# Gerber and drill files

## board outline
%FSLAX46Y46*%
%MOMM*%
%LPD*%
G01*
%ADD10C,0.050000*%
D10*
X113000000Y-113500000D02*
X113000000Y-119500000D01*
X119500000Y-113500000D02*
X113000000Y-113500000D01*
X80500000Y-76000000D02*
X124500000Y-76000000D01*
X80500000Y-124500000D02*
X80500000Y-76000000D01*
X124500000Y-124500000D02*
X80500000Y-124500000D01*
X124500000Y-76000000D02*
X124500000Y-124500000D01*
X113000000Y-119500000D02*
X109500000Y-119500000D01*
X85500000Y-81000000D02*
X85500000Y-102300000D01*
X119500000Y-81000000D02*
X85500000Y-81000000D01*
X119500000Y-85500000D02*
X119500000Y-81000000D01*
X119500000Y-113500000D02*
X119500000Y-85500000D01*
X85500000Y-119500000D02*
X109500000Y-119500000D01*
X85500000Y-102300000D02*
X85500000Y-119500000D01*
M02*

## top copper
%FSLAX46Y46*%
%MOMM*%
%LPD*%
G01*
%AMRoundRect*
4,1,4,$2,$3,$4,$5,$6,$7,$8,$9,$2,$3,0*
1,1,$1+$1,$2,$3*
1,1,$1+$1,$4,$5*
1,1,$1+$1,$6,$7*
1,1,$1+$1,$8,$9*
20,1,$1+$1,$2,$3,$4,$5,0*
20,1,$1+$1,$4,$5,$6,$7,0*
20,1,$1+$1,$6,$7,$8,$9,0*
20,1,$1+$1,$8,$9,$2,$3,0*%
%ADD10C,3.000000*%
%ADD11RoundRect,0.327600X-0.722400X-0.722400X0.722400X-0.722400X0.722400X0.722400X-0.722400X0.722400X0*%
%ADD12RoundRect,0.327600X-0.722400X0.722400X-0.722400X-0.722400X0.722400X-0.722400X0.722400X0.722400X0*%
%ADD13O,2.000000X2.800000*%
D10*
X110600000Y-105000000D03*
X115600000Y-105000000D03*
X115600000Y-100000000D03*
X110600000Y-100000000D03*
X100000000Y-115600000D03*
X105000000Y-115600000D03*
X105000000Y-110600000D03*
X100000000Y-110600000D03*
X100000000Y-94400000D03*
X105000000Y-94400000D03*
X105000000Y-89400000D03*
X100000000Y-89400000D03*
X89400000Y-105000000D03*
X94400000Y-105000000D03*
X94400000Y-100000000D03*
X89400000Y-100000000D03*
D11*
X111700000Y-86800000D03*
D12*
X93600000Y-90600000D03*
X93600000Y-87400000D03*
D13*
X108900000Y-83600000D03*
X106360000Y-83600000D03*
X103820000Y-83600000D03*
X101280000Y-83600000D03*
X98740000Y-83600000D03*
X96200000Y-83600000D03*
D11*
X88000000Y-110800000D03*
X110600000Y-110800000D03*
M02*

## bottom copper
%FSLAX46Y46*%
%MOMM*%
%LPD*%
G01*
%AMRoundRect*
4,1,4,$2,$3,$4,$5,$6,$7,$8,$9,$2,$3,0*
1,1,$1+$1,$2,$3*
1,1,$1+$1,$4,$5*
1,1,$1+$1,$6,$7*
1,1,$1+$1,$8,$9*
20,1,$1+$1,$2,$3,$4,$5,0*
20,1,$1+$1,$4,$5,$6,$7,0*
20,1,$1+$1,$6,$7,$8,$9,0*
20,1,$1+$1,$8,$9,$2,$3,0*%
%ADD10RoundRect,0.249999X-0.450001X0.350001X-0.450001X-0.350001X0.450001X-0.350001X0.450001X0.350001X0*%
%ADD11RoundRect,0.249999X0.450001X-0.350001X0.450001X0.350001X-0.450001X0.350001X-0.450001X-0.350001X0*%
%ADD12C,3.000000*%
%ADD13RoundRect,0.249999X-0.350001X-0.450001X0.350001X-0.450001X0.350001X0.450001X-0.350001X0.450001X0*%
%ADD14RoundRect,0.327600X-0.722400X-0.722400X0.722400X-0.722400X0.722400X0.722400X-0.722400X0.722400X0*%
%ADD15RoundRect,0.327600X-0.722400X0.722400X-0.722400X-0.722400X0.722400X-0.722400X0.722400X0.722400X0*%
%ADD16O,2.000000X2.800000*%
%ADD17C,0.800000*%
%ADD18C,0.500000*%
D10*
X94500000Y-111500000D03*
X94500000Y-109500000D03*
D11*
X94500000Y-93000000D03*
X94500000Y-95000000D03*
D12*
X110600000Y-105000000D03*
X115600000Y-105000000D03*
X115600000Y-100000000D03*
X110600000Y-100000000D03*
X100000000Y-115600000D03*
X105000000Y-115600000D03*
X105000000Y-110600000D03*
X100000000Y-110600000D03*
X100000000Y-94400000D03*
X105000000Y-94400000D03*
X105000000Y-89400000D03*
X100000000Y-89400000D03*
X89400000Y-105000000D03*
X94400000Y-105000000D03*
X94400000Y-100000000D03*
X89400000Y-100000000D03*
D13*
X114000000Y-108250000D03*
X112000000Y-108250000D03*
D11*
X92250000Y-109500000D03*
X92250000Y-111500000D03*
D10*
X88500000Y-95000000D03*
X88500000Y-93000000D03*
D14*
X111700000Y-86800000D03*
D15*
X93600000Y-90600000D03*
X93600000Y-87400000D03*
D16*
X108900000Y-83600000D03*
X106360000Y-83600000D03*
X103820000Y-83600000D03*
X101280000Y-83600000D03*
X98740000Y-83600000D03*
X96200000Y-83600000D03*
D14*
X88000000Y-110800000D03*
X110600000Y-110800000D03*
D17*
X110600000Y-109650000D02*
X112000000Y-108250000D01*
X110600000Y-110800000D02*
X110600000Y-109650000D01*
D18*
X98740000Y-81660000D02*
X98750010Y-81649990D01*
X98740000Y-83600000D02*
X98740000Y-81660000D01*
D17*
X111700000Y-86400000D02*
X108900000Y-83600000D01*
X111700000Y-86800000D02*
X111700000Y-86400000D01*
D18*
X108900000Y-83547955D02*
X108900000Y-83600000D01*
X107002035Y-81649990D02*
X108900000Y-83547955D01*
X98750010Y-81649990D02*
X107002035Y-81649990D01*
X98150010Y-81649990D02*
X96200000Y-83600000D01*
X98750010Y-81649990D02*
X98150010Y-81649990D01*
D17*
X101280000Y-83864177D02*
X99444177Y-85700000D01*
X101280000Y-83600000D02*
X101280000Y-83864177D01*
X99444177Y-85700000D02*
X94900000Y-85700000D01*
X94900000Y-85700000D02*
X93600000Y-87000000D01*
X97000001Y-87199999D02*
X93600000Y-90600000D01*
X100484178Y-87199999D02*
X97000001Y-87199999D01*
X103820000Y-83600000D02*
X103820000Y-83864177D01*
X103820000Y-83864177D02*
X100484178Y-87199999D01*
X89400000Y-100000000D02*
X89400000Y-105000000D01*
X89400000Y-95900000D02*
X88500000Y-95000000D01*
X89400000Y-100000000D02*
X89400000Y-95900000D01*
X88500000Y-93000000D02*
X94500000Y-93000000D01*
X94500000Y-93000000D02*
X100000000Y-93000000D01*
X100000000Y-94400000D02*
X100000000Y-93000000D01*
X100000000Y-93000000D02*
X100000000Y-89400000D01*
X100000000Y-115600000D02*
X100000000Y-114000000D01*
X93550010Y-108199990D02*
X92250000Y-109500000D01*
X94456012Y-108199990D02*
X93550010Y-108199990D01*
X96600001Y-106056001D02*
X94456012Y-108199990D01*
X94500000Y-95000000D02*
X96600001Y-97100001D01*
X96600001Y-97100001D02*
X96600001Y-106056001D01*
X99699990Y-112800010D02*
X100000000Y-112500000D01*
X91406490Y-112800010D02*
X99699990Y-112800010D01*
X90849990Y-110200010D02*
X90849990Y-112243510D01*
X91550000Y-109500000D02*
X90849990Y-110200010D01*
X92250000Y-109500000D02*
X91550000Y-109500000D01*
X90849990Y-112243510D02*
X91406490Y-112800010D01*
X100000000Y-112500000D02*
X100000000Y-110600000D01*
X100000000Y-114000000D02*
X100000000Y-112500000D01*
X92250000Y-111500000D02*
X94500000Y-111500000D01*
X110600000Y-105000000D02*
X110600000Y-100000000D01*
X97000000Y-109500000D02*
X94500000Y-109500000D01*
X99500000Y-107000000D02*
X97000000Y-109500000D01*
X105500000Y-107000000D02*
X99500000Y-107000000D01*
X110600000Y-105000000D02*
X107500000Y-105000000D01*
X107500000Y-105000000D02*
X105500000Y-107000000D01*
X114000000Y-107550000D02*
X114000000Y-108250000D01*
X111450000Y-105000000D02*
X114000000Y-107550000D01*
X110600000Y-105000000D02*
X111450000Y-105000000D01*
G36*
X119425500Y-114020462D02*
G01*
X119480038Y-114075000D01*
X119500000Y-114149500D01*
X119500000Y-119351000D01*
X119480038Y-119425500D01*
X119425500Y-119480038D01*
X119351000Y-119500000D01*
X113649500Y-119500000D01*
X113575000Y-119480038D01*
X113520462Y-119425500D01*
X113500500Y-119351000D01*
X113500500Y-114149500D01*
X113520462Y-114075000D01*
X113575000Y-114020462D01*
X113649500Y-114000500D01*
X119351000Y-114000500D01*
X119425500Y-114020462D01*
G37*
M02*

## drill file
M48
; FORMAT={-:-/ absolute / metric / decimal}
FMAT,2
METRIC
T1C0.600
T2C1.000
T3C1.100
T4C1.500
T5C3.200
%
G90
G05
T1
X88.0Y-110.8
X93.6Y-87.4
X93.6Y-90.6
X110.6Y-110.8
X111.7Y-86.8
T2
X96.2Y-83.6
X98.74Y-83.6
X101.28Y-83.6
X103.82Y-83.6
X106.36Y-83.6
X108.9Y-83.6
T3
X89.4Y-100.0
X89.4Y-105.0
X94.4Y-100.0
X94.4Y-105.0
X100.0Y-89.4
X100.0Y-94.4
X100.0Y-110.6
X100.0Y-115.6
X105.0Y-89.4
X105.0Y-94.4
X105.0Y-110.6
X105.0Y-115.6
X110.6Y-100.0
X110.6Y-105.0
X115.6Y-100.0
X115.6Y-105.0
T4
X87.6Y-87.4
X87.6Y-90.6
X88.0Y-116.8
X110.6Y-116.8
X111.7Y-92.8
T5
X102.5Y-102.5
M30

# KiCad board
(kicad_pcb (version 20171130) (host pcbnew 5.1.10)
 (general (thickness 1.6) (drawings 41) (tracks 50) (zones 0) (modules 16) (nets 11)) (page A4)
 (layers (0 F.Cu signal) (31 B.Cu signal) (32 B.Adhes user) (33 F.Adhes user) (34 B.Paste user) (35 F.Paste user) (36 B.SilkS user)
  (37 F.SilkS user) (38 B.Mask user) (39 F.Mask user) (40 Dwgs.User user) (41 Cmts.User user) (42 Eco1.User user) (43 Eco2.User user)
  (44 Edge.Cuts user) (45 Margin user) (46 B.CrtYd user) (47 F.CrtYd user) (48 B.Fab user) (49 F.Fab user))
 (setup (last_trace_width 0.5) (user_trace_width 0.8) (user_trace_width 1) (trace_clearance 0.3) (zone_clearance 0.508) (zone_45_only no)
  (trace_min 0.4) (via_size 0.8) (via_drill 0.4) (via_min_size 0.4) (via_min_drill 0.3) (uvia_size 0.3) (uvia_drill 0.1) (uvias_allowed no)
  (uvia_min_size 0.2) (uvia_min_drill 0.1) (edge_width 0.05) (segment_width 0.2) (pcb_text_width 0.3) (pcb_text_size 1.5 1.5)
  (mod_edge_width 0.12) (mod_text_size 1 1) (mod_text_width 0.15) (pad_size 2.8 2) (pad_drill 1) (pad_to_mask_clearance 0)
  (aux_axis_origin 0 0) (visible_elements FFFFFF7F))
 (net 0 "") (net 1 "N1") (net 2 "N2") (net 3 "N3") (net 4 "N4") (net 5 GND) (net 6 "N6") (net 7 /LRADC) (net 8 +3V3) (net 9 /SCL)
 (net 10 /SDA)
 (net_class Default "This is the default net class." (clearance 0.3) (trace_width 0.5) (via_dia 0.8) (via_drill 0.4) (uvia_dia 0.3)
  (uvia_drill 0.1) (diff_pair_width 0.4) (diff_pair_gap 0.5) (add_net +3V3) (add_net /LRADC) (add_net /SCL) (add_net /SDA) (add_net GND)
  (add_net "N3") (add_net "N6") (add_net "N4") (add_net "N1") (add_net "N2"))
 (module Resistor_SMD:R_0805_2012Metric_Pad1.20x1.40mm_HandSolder (layer B.Cu) (at 94.5 110.5 270)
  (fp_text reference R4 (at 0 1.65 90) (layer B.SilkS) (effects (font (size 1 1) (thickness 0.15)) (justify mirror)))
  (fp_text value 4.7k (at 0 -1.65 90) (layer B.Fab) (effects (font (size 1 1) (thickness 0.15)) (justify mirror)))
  (pad 2 smd roundrect (at 1 0 270) (size 1.2 1.4) (layers B.Cu B.Paste B.Mask) (roundrect_rratio 0.2083325) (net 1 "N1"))
  (pad 1 smd roundrect (at -1 0 270) (size 1.2 1.4) (layers B.Cu B.Paste B.Mask) (roundrect_rratio 0.2083325) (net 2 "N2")))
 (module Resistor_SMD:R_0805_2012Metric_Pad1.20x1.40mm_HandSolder (layer B.Cu) (at 94.5 94 90)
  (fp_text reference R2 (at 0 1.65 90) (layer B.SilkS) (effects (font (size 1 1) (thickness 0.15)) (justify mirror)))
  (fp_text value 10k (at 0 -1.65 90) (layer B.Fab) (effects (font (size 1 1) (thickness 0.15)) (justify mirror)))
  (pad 2 smd roundrect (at 1 0 90) (size 1.2 1.4) (layers B.Cu B.Paste B.Mask) (roundrect_rratio 0.2083325) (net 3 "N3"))
  (pad 1 smd roundrect (at -1 0 90) (size 1.2 1.4) (layers B.Cu B.Paste B.Mask) (roundrect_rratio 0.2083325) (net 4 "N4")))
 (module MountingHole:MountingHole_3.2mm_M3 (layer F.Cu) (at 102.5 102.5)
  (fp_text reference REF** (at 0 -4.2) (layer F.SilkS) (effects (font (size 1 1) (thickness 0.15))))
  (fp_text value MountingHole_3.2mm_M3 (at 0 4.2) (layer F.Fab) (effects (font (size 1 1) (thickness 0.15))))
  (pad 1 np_thru_hole circle (at 0 0) (size 3.2 3.2) (drill 3.2) (layers *.Cu *.Mask)))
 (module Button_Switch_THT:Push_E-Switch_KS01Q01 (layer F.Cu) (at 110.6 100)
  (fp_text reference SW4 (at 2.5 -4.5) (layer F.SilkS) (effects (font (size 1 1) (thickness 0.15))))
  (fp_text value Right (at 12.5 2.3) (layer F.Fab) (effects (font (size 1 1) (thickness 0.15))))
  (pad 3 thru_hole circle (at 0 5) (size 3 3) (drill 1.1) (layers *.Cu *.Mask) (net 2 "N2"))
  (pad 4 thru_hole circle (at 5 5) (size 3 3) (drill 1.1) (layers *.Cu *.Mask) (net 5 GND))
  (pad 2 thru_hole circle (at 5 0) (size 3 3) (drill 1.1) (layers *.Cu *.Mask) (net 5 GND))
  (pad 1 thru_hole circle (at 0 0) (size 3 3) (drill 1.1) (layers *.Cu *.Mask) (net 2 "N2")))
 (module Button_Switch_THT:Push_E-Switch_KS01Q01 (layer F.Cu) (at 100 110.6)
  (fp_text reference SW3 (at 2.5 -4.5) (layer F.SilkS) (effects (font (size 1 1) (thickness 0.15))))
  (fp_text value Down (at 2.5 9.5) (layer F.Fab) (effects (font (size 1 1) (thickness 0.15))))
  (pad 3 thru_hole circle (at 0 5) (size 3 3) (drill 1.1) (layers *.Cu *.Mask) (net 4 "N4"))
  (pad 4 thru_hole circle (at 5 5) (size 3 3) (drill 1.1) (layers *.Cu *.Mask) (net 5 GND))
  (pad 2 thru_hole circle (at 5 0) (size 3 3) (drill 1.1) (layers *.Cu *.Mask) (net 5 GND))
  (pad 1 thru_hole circle (at 0 0) (size 3 3) (drill 1.1) (layers *.Cu *.Mask) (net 4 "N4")))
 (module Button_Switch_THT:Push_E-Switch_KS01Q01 (layer F.Cu) (at 100 89.4)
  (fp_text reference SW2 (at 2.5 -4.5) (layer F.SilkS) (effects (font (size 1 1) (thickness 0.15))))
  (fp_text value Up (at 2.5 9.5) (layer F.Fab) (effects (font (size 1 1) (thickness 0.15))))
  (pad 3 thru_hole circle (at 0 5) (size 3 3) (drill 1.1) (layers *.Cu *.Mask) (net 3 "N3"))
  (pad 4 thru_hole circle (at 5 5) (size 3 3) (drill 1.1) (layers *.Cu *.Mask) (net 5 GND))
  (pad 2 thru_hole circle (at 5 0) (size 3 3) (drill 1.1) (layers *.Cu *.Mask) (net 5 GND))
  (pad 1 thru_hole circle (at 0 0) (size 3 3) (drill 1.1) (layers *.Cu *.Mask) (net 3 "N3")))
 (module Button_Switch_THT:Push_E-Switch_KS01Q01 (layer F.Cu) (at 89.4 100)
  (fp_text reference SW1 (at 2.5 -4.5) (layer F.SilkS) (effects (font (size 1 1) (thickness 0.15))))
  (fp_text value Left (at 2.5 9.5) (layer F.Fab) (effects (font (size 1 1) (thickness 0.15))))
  (pad 3 thru_hole circle (at 0 5) (size 3 3) (drill 1.1) (layers *.Cu *.Mask) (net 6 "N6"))
  (pad 4 thru_hole circle (at 5 5) (size 3 3) (drill 1.1) (layers *.Cu *.Mask) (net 5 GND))
  (pad 2 thru_hole circle (at 5 0) (size 3 3) (drill 1.1) (layers *.Cu *.Mask) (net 5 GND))
  (pad 1 thru_hole circle (at 0 0) (size 3 3) (drill 1.1) (layers *.Cu *.Mask) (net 6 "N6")))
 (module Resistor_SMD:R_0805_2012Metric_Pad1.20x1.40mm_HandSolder (layer B.Cu) (at 113 108.25)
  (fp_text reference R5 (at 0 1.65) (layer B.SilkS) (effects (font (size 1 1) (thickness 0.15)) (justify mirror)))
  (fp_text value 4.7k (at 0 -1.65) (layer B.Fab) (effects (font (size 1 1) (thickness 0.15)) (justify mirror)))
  (pad 2 smd roundrect (at 1 0) (size 1.2 1.4) (layers B.Cu B.Paste B.Mask) (roundrect_rratio 0.2083325) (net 2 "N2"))
  (pad 1 smd roundrect (at -1 0) (size 1.2 1.4) (layers B.Cu B.Paste B.Mask) (roundrect_rratio 0.2083325) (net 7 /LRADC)))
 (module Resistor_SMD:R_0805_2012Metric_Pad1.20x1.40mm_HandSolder (layer B.Cu) (at 92.25 110.5 90)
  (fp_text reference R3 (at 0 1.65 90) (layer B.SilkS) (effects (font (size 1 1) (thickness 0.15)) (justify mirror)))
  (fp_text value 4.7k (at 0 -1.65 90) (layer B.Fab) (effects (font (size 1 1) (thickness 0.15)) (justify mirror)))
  (pad 2 smd roundrect (at 1 0 90) (size 1.2 1.4) (layers B.Cu B.Paste B.Mask) (roundrect_rratio 0.2083325) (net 4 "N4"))
  (pad 1 smd roundrect (at -1 0 90) (size 1.2 1.4) (layers B.Cu B.Paste B.Mask) (roundrect_rratio 0.2083325) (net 1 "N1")))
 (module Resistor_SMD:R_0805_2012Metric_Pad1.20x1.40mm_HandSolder (layer B.Cu) (at 88.5 94 270)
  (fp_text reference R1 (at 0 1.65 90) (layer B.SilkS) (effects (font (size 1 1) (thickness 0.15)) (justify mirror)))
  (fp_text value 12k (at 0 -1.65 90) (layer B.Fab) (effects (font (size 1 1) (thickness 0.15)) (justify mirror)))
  (pad 2 smd roundrect (at 1 0 270) (size 1.2 1.4) (layers B.Cu B.Paste B.Mask) (roundrect_rratio 0.2083325) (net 6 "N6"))
  (pad 1 smd roundrect (at -1 0 270) (size 1.2 1.4) (layers B.Cu B.Paste B.Mask) (roundrect_rratio 0.2083325) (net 3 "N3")))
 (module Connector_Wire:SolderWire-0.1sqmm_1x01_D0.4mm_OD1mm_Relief (layer F.Cu) (at 111.7 86.8)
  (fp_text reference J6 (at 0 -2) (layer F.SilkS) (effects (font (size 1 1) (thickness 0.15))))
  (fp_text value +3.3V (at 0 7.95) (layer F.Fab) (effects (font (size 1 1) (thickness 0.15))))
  (pad "" np_thru_hole circle (at 0 6) (size 1.5 1.5) (drill 1.5) (layers *.Cu *.Mask))
  (pad 1 thru_hole roundrect (at 0 0) (size 2.1 2.1) (drill 0.6) (layers *.Cu *.Mask) (roundrect_rratio 0.156) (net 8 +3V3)))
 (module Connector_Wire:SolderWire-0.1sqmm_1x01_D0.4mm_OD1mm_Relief (layer F.Cu) (at 93.6 90.6 270)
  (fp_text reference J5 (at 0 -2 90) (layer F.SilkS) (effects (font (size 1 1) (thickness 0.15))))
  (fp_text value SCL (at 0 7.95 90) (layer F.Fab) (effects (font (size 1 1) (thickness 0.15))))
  (pad "" np_thru_hole circle (at 0 6 270) (size 1.5 1.5) (drill 1.5) (layers *.Cu *.Mask))
  (pad 1 thru_hole roundrect (at 0 0 270) (size 2.1 2.1) (drill 0.6) (layers *.Cu *.Mask) (roundrect_rratio 0.156) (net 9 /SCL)))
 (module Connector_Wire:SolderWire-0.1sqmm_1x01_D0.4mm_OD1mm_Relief (layer F.Cu) (at 93.6 87.4 270)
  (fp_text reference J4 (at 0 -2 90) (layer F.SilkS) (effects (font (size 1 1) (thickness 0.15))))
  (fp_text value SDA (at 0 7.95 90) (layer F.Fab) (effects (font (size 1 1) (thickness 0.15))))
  (pad "" np_thru_hole circle (at 0 6 270) (size 1.5 1.5) (drill 1.5) (layers *.Cu *.Mask))
  (pad 1 thru_hole roundrect (at 0 0 270) (size 2.1 2.1) (drill 0.6) (layers *.Cu *.Mask) (roundrect_rratio 0.156) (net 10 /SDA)))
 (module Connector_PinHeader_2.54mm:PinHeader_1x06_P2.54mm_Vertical (layer B.Cu) (at 108.9 83.6 90)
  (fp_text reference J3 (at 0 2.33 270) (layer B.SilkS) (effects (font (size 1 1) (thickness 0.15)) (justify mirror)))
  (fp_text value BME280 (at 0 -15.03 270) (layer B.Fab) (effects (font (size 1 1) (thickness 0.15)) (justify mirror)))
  (pad 1 thru_hole oval (at 0 0 90) (size 2.8 2) (drill 1) (layers *.Cu *.Mask) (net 8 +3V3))
  (pad 2 thru_hole oval (at 0 -2.54 90) (size 2.8 2) (drill 1) (layers *.Cu *.Mask) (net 5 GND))
  (pad 3 thru_hole oval (at 0 -5.08 90) (size 2.8 2) (drill 1) (layers *.Cu *.Mask) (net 9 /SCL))
  (pad 4 thru_hole oval (at 0 -7.62 90) (size 2.8 2) (drill 1) (layers *.Cu *.Mask) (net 10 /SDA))
  (pad 5 thru_hole oval (at 0 -10.16 90) (size 2.8 2) (drill 1) (layers *.Cu *.Mask) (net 8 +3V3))
  (pad 6 thru_hole oval (at 0 -12.7 90) (size 2.8 2) (drill 1) (layers *.Cu *.Mask) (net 8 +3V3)))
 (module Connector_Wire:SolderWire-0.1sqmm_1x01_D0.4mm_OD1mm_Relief (layer F.Cu) (at 88 110.8)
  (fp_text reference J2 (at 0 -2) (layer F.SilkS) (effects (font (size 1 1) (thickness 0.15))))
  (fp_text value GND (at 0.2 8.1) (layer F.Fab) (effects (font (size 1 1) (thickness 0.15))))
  (pad "" np_thru_hole circle (at 0 6) (size 1.5 1.5) (drill 1.5) (layers *.Cu *.Mask))
  (pad 1 thru_hole roundrect (at 0 0) (size 2.1 2.1) (drill 0.6) (layers *.Cu *.Mask) (roundrect_rratio 0.156) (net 5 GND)))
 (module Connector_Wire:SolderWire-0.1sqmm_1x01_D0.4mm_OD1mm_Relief (layer F.Cu) (at 110.6 110.8)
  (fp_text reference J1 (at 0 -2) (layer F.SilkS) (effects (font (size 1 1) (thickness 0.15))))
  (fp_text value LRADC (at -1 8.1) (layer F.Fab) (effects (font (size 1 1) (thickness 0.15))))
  (pad "" np_thru_hole circle (at 0 6) (size 1.5 1.5) (drill 1.5) (layers *.Cu *.Mask))
  (pad 1 thru_hole roundrect (at 0 0) (size 2.1 2.1) (drill 0.6) (layers *.Cu *.Mask) (roundrect_rratio 0.156) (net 7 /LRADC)))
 (gr_line (start 113 113.5) (end 113 119.5) (layer Edge.Cuts) (width 0.05))
 (gr_line (start 119.5 113.5) (end 113 113.5) (layer Edge.Cuts) (width 0.05))
 (gr_line (start 80.5 76) (end 124.5 76) (layer Edge.Cuts) (width 0.05))
 (gr_line (start 80.5 124.5) (end 80.5 76) (layer Edge.Cuts) (width 0.05))
 (gr_line (start 124.5 124.5) (end 80.5 124.5) (layer Edge.Cuts) (width 0.05))
 (gr_line (start 124.5 76) (end 124.5 124.5) (layer Edge.Cuts) (width 0.05))
 (gr_line (start 113 119.5) (end 109.5 119.5) (layer Edge.Cuts) (width 0.05))
 (gr_line (start 85.5 81) (end 85.5 102.3) (layer Edge.Cuts) (width 0.05))
 (gr_line (start 119.5 81) (end 85.5 81) (layer Edge.Cuts) (width 0.05))
 (gr_line (start 119.5 85.5) (end 119.5 81) (layer Edge.Cuts) (width 0.05))
 (gr_line (start 119.5 113.5) (end 119.5 85.5) (layer Edge.Cuts) (width 0.05))
 (gr_line (start 85.5 119.5) (end 109.5 119.5) (layer Edge.Cuts) (width 0.05))
 (gr_line (start 85.5 102.3) (end 85.5 119.5) (layer Edge.Cuts) (width 0.05))
 (segment (start 110.6 109.65) (end 112 108.25) (width 0.8) (layer B.Cu) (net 7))
 (segment (start 110.6 110.8) (end 110.6 109.65) (width 0.8) (layer B.Cu) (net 7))
 (segment (start 98.74 81.66) (end 98.75001 81.64999) (width 0.5) (layer B.Cu) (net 8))
 (segment (start 98.74 83.6) (end 98.74 81.66) (width 0.5) (layer B.Cu) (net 8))
 (segment (start 111.7 86.4) (end 108.9 83.6) (width 0.8) (layer B.Cu) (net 8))
 (segment (start 111.7 86.8) (end 111.7 86.4) (width 0.8) (layer B.Cu) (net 8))
 (segment (start 108.9 83.547955) (end 108.9 83.6) (width 0.5) (layer B.Cu) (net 8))
 (segment (start 107.002035 81.64999) (end 108.9 83.547955) (width 0.5) (layer B.Cu) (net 8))
 (segment (start 98.75001 81.64999) (end 107.002035 81.64999) (width 0.5) (layer B.Cu) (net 8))
 (segment (start 98.15001 81.64999) (end 96.2 83.6) (width 0.5) (layer B.Cu) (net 8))
 (segment (start 98.75001 81.64999) (end 98.15001 81.64999) (width 0.5) (layer B.Cu) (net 8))
 (segment (start 101.28 83.864177) (end 99.444177 85.7) (width 0.8) (layer B.Cu) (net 10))
 (segment (start 101.28 83.6) (end 101.28 83.864177) (width 0.8) (layer B.Cu) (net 10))
 (segment (start 99.444177 85.7) (end 94.9 85.7) (width 0.8) (layer B.Cu) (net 10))
 (segment (start 94.9 85.7) (end 93.6 87) (width 0.8) (layer B.Cu) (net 10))
 (segment (start 97.000001 87.199999) (end 93.6 90.6) (width 0.8) (layer B.Cu) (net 9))
 (segment (start 100.484178 87.199999) (end 97.000001 87.199999) (width 0.8) (layer B.Cu) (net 9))
 (segment (start 103.82 83.6) (end 103.82 83.864177) (width 0.8) (layer B.Cu) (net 9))
 (segment (start 103.82 83.864177) (end 100.484178 87.199999) (width 0.8) (layer B.Cu) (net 9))
 (segment (start 89.4 100) (end 89.4 105) (width 0.8) (layer B.Cu) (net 6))
 (segment (start 89.4 95.9) (end 88.5 95) (width 0.8) (layer B.Cu) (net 6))
 (segment (start 89.4 100) (end 89.4 95.9) (width 0.8) (layer B.Cu) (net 6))
 (segment (start 88.5 93) (end 94.5 93) (width 0.8) (layer B.Cu) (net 3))
 (segment (start 94.5 93) (end 100 93) (width 0.8) (layer B.Cu) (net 3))
 (segment (start 100 94.4) (end 100 93) (width 0.8) (layer B.Cu) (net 3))
 (segment (start 100 93) (end 100 89.4) (width 0.8) (layer B.Cu) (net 3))
 (segment (start 100 115.6) (end 100 114) (width 0.8) (layer B.Cu) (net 4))
 (segment (start 93.55001 108.19999) (end 92.25 109.5) (width 0.8) (layer B.Cu) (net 4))
 (segment (start 94.456012 108.19999) (end 93.55001 108.19999) (width 0.8) (layer B.Cu) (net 4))
 (segment (start 96.600001 106.056001) (end 94.456012 108.19999) (width 0.8) (layer B.Cu) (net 4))
 (segment (start 94.5 95) (end 96.600001 97.100001) (width 0.8) (layer B.Cu) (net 4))
 (segment (start 96.600001 97.100001) (end 96.600001 106.056001) (width 0.8) (layer B.Cu) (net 4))
 (segment (start 99.69999 112.80001) (end 100 112.5) (width 0.8) (layer B.Cu) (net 4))
 (segment (start 91.40649 112.80001) (end 99.69999 112.80001) (width 0.8) (layer B.Cu) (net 4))
 (segment (start 90.84999 110.20001) (end 90.84999 112.24351) (width 0.8) (layer B.Cu) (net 4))
 (segment (start 91.55 109.5) (end 90.84999 110.20001) (width 0.8) (layer B.Cu) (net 4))
 (segment (start 92.25 109.5) (end 91.55 109.5) (width 0.8) (layer B.Cu) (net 4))
 (segment (start 90.84999 112.24351) (end 91.40649 112.80001) (width 0.8) (layer B.Cu) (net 4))
 (segment (start 100 112.5) (end 100 110.6) (width 0.8) (layer B.Cu) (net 4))
 (segment (start 100 114) (end 100 112.5) (width 0.8) (layer B.Cu) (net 4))
 (segment (start 92.25 111.5) (end 94.5 111.5) (width 0.8) (layer B.Cu) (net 1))
 (segment (start 110.6 105) (end 110.6 100) (width 0.8) (layer B.Cu) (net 2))
 (segment (start 97 109.5) (end 94.5 109.5) (width 0.8) (layer B.Cu) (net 2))
 (segment (start 99.5 107) (end 97 109.5) (width 0.8) (layer B.Cu) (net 2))
 (segment (start 105.5 107) (end 99.5 107) (width 0.8) (layer B.Cu) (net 2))
 (segment (start 110.6 105) (end 107.5 105) (width 0.8) (layer B.Cu) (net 2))
 (segment (start 107.5 105) (end 105.5 107) (width 0.8) (layer B.Cu) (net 2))
 (segment (start 114 107.55) (end 114 108.25) (width 0.8) (layer B.Cu) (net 2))
 (segment (start 111.45 105) (end 114 107.55) (width 0.8) (layer B.Cu) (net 2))
 (segment (start 110.6 105) (end 111.45 105) (width 0.8) (layer B.Cu) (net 2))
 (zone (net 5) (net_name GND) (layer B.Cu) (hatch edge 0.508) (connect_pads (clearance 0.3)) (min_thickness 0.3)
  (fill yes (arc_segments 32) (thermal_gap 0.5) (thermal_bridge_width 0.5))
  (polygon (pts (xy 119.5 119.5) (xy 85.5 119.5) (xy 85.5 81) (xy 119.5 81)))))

